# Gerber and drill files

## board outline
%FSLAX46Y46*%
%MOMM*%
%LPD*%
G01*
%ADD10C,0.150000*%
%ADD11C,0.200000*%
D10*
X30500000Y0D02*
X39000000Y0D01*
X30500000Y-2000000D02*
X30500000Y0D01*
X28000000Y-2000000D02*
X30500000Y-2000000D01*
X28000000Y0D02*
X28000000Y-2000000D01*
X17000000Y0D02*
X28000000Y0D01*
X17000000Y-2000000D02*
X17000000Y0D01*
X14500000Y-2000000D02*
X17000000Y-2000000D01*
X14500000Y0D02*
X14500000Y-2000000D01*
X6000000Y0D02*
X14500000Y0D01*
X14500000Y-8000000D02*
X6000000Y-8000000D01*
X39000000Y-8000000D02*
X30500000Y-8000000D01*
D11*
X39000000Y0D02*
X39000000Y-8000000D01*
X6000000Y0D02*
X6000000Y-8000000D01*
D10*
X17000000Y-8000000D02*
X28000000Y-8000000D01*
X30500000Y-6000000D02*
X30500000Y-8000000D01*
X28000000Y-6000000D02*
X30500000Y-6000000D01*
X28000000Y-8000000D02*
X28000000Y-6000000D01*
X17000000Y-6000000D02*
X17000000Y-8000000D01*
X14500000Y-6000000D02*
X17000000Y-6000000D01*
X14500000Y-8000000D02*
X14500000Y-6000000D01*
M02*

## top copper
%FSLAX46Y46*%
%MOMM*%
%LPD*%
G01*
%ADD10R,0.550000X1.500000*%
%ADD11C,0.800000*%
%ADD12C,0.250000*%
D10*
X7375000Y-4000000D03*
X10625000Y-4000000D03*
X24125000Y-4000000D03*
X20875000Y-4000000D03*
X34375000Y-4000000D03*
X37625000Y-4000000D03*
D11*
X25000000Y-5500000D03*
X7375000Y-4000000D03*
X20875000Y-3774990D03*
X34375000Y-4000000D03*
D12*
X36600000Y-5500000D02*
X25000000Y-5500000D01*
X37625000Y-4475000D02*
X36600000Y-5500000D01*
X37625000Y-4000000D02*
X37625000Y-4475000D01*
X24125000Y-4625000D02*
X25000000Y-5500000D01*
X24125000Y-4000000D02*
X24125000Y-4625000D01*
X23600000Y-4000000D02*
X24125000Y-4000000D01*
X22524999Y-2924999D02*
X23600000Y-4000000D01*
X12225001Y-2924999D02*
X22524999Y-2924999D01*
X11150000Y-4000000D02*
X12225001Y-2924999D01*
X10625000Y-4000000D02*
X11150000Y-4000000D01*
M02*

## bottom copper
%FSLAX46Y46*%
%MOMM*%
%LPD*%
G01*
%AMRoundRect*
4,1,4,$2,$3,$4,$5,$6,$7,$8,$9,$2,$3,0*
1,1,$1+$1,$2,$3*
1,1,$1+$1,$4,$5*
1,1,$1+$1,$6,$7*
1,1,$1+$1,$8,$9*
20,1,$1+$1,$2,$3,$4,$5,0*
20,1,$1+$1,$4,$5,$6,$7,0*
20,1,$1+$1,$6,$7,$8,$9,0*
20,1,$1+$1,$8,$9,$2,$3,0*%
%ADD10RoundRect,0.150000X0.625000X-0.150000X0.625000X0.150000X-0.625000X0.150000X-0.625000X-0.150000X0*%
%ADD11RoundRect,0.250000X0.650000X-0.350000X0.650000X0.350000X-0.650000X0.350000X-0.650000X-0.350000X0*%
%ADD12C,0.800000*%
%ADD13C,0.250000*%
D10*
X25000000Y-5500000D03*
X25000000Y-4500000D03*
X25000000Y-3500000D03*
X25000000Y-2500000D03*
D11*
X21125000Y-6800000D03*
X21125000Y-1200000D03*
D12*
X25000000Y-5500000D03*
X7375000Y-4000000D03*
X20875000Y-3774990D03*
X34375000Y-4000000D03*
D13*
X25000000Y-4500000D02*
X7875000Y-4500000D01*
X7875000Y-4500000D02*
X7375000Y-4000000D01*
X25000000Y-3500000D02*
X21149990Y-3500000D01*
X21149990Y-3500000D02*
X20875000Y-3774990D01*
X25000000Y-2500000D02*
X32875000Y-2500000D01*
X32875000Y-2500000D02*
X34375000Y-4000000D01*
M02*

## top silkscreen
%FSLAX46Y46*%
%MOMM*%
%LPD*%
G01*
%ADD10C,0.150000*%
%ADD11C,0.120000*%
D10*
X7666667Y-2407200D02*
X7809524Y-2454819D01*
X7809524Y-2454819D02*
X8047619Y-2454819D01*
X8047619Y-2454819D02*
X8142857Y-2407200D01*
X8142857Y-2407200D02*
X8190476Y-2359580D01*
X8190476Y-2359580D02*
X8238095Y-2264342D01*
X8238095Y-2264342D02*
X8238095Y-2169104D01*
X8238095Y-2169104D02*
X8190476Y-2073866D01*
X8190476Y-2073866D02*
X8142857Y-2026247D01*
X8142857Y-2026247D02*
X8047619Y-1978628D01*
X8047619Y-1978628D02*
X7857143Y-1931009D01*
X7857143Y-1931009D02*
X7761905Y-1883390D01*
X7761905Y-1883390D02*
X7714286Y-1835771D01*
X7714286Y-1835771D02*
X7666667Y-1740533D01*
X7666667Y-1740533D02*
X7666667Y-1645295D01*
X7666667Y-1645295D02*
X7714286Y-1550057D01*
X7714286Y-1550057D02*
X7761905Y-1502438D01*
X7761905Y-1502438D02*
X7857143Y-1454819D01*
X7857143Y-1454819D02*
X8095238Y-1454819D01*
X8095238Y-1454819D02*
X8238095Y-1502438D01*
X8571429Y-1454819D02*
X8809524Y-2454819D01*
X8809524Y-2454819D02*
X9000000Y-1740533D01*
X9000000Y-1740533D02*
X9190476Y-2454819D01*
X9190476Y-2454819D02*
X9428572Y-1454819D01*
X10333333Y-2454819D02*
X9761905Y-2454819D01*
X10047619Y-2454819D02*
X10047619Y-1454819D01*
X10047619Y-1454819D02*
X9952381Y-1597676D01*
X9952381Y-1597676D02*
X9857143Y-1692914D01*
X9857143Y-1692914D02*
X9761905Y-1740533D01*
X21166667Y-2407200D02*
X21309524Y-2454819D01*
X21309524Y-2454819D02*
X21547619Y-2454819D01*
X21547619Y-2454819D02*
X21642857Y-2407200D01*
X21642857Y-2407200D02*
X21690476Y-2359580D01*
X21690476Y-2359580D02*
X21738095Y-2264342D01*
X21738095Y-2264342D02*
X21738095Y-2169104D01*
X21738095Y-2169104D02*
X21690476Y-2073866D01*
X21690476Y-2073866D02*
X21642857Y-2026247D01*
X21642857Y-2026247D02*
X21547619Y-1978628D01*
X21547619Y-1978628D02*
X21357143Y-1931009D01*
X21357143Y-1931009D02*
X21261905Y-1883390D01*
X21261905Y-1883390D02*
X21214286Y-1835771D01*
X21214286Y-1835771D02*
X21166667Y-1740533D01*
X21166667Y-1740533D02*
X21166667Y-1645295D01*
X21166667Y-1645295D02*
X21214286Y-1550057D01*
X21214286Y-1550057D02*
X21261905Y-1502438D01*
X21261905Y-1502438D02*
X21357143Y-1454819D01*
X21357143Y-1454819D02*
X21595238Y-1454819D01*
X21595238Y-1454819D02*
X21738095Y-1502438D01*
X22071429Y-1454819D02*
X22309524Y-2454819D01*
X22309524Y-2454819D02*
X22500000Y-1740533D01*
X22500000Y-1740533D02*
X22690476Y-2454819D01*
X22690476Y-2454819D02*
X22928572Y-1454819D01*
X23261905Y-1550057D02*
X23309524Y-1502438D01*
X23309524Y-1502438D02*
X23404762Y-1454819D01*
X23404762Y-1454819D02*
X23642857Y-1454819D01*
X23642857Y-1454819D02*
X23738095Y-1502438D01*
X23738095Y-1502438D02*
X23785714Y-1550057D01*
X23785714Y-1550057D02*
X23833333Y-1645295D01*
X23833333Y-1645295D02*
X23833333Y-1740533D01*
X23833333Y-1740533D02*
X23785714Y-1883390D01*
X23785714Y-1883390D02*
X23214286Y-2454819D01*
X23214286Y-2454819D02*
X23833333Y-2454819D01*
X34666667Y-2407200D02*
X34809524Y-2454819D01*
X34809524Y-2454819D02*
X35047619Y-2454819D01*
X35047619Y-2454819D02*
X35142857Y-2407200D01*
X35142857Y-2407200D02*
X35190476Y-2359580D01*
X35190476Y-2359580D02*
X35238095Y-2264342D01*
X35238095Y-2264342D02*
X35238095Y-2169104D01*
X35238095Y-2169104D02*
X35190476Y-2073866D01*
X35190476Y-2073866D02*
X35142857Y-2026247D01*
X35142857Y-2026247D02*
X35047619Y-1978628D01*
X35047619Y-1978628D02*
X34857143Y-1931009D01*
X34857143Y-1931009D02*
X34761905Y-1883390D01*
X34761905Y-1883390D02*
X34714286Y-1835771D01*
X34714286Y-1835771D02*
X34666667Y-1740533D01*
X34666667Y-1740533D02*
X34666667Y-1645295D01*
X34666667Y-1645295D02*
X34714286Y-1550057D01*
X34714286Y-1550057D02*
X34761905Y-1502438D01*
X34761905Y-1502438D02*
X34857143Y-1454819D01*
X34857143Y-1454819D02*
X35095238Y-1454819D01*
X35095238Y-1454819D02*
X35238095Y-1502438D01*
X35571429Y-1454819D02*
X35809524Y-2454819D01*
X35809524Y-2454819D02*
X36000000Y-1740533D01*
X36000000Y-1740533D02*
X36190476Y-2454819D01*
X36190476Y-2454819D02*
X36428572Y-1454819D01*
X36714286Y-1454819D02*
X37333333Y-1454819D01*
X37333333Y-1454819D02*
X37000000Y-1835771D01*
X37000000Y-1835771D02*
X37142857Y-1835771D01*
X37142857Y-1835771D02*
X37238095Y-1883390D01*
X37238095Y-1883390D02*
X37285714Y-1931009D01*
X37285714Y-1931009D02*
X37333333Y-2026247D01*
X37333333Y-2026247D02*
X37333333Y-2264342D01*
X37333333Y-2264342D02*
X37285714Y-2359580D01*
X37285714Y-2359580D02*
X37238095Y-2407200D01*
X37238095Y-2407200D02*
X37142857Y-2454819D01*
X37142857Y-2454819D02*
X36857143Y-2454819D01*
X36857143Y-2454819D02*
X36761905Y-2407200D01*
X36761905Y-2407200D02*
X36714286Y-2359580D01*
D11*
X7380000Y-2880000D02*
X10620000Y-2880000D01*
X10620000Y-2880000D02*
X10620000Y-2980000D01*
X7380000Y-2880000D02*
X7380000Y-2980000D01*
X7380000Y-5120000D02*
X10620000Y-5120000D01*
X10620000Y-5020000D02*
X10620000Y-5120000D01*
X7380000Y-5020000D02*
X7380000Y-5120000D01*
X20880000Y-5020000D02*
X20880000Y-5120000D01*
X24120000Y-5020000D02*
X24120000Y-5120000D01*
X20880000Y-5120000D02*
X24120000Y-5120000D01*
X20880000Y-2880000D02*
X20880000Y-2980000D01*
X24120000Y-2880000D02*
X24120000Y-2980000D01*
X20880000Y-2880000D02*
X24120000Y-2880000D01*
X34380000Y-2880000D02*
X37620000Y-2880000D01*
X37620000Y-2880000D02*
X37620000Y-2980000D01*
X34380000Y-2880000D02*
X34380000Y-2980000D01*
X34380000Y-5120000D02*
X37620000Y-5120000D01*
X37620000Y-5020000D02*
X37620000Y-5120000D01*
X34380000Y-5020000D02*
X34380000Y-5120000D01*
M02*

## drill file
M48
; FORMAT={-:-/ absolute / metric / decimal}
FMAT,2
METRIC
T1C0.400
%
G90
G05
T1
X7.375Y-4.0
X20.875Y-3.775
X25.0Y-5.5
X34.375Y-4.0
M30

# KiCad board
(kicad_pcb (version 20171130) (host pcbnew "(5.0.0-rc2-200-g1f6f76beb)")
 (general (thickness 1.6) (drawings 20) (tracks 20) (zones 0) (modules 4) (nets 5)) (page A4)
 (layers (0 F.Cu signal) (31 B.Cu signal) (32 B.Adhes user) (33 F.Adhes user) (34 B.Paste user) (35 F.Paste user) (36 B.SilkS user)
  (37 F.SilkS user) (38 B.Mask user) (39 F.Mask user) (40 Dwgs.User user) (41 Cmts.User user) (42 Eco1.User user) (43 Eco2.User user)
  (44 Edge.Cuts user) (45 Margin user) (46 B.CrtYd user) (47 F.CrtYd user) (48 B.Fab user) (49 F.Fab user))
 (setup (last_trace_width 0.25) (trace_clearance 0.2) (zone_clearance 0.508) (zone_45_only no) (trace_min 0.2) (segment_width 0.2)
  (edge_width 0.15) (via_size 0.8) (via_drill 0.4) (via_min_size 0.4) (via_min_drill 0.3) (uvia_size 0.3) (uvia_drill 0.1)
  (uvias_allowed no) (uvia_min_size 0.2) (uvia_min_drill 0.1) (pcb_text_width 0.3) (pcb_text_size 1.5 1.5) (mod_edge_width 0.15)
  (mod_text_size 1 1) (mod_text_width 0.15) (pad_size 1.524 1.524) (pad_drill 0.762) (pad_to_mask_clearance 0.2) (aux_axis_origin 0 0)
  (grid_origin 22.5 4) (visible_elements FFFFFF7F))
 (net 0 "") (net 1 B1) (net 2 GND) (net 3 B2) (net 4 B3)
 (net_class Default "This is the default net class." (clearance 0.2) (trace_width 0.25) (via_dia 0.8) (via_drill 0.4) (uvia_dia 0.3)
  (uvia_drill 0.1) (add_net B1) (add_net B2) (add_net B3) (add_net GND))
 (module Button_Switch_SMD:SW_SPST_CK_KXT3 (layer F.Cu) (at 9 4)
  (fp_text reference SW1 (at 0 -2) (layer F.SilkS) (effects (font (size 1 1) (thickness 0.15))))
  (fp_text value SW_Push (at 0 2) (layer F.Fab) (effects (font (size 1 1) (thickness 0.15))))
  (fp_line (start -1.62 -1.12) (end 1.62 -1.12) (layer F.SilkS) (width 0.12))
  (fp_line (start 1.62 -1.12) (end 1.62 -1.02) (layer F.SilkS) (width 0.12))
  (fp_line (start -1.62 -1.12) (end -1.62 -1.02) (layer F.SilkS) (width 0.12))
  (fp_line (start -1.62 1.12) (end 1.62 1.12) (layer F.SilkS) (width 0.12))
  (fp_line (start 1.62 1.02) (end 1.62 1.12) (layer F.SilkS) (width 0.12))
  (fp_line (start -1.62 1.02) (end -1.62 1.12) (layer F.SilkS) (width 0.12))
  (pad 1 smd rect (at -1.625 0) (size 0.55 1.5) (layers F.Cu F.Paste F.Mask) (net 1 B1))
  (pad 2 smd rect (at 1.625 0) (size 0.55 1.5) (layers F.Cu F.Paste F.Mask) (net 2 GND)))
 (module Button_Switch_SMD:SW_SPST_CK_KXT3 (layer F.Cu) (at 22.5 4)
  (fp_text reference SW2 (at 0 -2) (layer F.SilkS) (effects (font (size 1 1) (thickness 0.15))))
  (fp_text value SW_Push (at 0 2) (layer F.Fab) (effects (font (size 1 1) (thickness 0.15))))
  (fp_line (start -1.62 1.02) (end -1.62 1.12) (layer F.SilkS) (width 0.12))
  (fp_line (start 1.62 1.02) (end 1.62 1.12) (layer F.SilkS) (width 0.12))
  (fp_line (start -1.62 1.12) (end 1.62 1.12) (layer F.SilkS) (width 0.12))
  (fp_line (start -1.62 -1.12) (end -1.62 -1.02) (layer F.SilkS) (width 0.12))
  (fp_line (start 1.62 -1.12) (end 1.62 -1.02) (layer F.SilkS) (width 0.12))
  (fp_line (start -1.62 -1.12) (end 1.62 -1.12) (layer F.SilkS) (width 0.12))
  (pad 2 smd rect (at 1.625 0) (size 0.55 1.5) (layers F.Cu F.Paste F.Mask) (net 2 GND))
  (pad 1 smd rect (at -1.625 0) (size 0.55 1.5) (layers F.Cu F.Paste F.Mask) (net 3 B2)))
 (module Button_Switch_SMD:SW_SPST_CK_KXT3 (layer F.Cu) (at 36 4)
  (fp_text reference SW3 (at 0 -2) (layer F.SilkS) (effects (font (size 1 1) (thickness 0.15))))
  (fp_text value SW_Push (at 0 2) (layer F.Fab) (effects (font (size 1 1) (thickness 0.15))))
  (fp_line (start -1.62 -1.12) (end 1.62 -1.12) (layer F.SilkS) (width 0.12))
  (fp_line (start 1.62 -1.12) (end 1.62 -1.02) (layer F.SilkS) (width 0.12))
  (fp_line (start -1.62 -1.12) (end -1.62 -1.02) (layer F.SilkS) (width 0.12))
  (fp_line (start -1.62 1.12) (end 1.62 1.12) (layer F.SilkS) (width 0.12))
  (fp_line (start 1.62 1.02) (end 1.62 1.12) (layer F.SilkS) (width 0.12))
  (fp_line (start -1.62 1.02) (end -1.62 1.12) (layer F.SilkS) (width 0.12))
  (pad 1 smd rect (at -1.625 0) (size 0.55 1.5) (layers F.Cu F.Paste F.Mask) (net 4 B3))
  (pad 2 smd rect (at 1.625 0) (size 0.55 1.5) (layers F.Cu F.Paste F.Mask) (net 2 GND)))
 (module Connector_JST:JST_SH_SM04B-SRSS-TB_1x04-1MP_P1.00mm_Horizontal (layer B.Cu) (at 23 4 90)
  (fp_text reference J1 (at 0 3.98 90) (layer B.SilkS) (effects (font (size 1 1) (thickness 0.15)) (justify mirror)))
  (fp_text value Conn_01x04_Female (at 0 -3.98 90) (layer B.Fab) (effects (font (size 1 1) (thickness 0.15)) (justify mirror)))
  (pad 1 smd roundrect (at -1.5 2 90) (size 0.6 1.55) (layers B.Cu B.Paste B.Mask) (roundrect_rratio 0.25) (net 2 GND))
  (pad 2 smd roundrect (at -0.5 2 90) (size 0.6 1.55) (layers B.Cu B.Paste B.Mask) (roundrect_rratio 0.25) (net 1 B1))
  (pad 3 smd roundrect (at 0.5 2 90) (size 0.6 1.55) (layers B.Cu B.Paste B.Mask) (roundrect_rratio 0.25) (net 3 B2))
  (pad 4 smd roundrect (at 1.5 2 90) (size 0.6 1.55) (layers B.Cu B.Paste B.Mask) (roundrect_rratio 0.25) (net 4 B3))
  (pad MP smd roundrect (at -2.8 -1.875 90) (size 1.2 1.8) (layers B.Cu B.Paste B.Mask) (roundrect_rratio 0.208333))
  (pad MP smd roundrect (at 2.8 -1.875 90) (size 1.2 1.8) (layers B.Cu B.Paste B.Mask) (roundrect_rratio 0.208333)))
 (gr_line (start 30.5 0) (end 39 0) (layer Edge.Cuts) (width 0.15))
 (gr_line (start 30.5 2) (end 30.5 0) (layer Edge.Cuts) (width 0.15))
 (gr_line (start 28 2) (end 30.5 2) (layer Edge.Cuts) (width 0.15))
 (gr_line (start 28 0) (end 28 2) (layer Edge.Cuts) (width 0.15))
 (gr_line (start 17 0) (end 28 0) (layer Edge.Cuts) (width 0.15))
 (gr_line (start 17 2) (end 17 0) (layer Edge.Cuts) (width 0.15))
 (gr_line (start 14.5 2) (end 17 2) (layer Edge.Cuts) (width 0.15))
 (gr_line (start 14.5 0) (end 14.5 2) (layer Edge.Cuts) (width 0.15))
 (gr_line (start 6 0) (end 14.5 0) (layer Edge.Cuts) (width 0.15))
 (gr_line (start 14.5 8) (end 6 8) (layer Edge.Cuts) (width 0.15))
 (gr_line (start 39 8) (end 30.5 8) (layer Edge.Cuts) (width 0.15))
 (gr_line (start 39 0) (end 39 8) (layer Edge.Cuts) (width 0.2))
 (gr_line (start 6 0) (end 6 8) (layer Edge.Cuts) (width 0.2))
 (gr_line (start 17 8) (end 28 8) (layer Edge.Cuts) (width 0.15))
 (gr_line (start 30.5 6) (end 30.5 8) (layer Edge.Cuts) (width 0.15))
 (gr_line (start 28 6) (end 30.5 6) (layer Edge.Cuts) (width 0.15))
 (gr_line (start 28 8) (end 28 6) (layer Edge.Cuts) (width 0.15))
 (gr_line (start 17 6) (end 17 8) (layer Edge.Cuts) (width 0.15))
 (gr_line (start 14.5 6) (end 17 6) (layer Edge.Cuts) (width 0.15))
 (gr_line (start 14.5 8) (end 14.5 6) (layer Edge.Cuts) (width 0.15))
 (via (at 25 5.5) (size 0.8) (drill 0.4) (layers F.Cu B.Cu) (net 2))
 (segment (start 36.6 5.5) (end 25 5.5) (width 0.25) (layer F.Cu) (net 2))
 (segment (start 37.625 4.475) (end 36.6 5.5) (width 0.25) (layer F.Cu) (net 2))
 (segment (start 37.625 4) (end 37.625 4.475) (width 0.25) (layer F.Cu) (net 2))
 (segment (start 24.125 4.625) (end 25 5.5) (width 0.25) (layer F.Cu) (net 2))
 (segment (start 24.125 4) (end 24.125 4.625) (width 0.25) (layer F.Cu) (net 2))
 (segment (start 23.6 4) (end 24.125 4) (width 0.25) (layer F.Cu) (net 2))
 (segment (start 22.524999 2.924999) (end 23.6 4) (width 0.25) (layer F.Cu) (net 2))
 (segment (start 12.225001 2.924999) (end 22.524999 2.924999) (width 0.25) (layer F.Cu) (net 2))
 (segment (start 11.15 4) (end 12.225001 2.924999) (width 0.25) (layer F.Cu) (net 2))
 (segment (start 10.625 4) (end 11.15 4) (width 0.25) (layer F.Cu) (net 2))
 (via (at 7.375 4) (size 0.8) (drill 0.4) (layers F.Cu B.Cu) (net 1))
 (segment (start 25 4.5) (end 7.875 4.5) (width 0.25) (layer B.Cu) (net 1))
 (segment (start 7.875 4.5) (end 7.375 4) (width 0.25) (layer B.Cu) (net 1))
 (segment (start 25 3.5) (end 21.14999 3.5) (width 0.25) (layer B.Cu) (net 3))
 (segment (start 21.14999 3.5) (end 20.875 3.77499) (width 0.25) (layer B.Cu) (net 3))
 (via (at 20.875 3.77499) (size 0.8) (drill 0.4) (layers F.Cu B.Cu) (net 3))
 (via (at 34.375 4) (size 0.8) (drill 0.4) (layers F.Cu B.Cu) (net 4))
 (segment (start 25 2.5) (end 32.875 2.5) (width 0.25) (layer B.Cu) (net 4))
 (segment (start 32.875 2.5) (end 34.375 4) (width 0.25) (layer B.Cu) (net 4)))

